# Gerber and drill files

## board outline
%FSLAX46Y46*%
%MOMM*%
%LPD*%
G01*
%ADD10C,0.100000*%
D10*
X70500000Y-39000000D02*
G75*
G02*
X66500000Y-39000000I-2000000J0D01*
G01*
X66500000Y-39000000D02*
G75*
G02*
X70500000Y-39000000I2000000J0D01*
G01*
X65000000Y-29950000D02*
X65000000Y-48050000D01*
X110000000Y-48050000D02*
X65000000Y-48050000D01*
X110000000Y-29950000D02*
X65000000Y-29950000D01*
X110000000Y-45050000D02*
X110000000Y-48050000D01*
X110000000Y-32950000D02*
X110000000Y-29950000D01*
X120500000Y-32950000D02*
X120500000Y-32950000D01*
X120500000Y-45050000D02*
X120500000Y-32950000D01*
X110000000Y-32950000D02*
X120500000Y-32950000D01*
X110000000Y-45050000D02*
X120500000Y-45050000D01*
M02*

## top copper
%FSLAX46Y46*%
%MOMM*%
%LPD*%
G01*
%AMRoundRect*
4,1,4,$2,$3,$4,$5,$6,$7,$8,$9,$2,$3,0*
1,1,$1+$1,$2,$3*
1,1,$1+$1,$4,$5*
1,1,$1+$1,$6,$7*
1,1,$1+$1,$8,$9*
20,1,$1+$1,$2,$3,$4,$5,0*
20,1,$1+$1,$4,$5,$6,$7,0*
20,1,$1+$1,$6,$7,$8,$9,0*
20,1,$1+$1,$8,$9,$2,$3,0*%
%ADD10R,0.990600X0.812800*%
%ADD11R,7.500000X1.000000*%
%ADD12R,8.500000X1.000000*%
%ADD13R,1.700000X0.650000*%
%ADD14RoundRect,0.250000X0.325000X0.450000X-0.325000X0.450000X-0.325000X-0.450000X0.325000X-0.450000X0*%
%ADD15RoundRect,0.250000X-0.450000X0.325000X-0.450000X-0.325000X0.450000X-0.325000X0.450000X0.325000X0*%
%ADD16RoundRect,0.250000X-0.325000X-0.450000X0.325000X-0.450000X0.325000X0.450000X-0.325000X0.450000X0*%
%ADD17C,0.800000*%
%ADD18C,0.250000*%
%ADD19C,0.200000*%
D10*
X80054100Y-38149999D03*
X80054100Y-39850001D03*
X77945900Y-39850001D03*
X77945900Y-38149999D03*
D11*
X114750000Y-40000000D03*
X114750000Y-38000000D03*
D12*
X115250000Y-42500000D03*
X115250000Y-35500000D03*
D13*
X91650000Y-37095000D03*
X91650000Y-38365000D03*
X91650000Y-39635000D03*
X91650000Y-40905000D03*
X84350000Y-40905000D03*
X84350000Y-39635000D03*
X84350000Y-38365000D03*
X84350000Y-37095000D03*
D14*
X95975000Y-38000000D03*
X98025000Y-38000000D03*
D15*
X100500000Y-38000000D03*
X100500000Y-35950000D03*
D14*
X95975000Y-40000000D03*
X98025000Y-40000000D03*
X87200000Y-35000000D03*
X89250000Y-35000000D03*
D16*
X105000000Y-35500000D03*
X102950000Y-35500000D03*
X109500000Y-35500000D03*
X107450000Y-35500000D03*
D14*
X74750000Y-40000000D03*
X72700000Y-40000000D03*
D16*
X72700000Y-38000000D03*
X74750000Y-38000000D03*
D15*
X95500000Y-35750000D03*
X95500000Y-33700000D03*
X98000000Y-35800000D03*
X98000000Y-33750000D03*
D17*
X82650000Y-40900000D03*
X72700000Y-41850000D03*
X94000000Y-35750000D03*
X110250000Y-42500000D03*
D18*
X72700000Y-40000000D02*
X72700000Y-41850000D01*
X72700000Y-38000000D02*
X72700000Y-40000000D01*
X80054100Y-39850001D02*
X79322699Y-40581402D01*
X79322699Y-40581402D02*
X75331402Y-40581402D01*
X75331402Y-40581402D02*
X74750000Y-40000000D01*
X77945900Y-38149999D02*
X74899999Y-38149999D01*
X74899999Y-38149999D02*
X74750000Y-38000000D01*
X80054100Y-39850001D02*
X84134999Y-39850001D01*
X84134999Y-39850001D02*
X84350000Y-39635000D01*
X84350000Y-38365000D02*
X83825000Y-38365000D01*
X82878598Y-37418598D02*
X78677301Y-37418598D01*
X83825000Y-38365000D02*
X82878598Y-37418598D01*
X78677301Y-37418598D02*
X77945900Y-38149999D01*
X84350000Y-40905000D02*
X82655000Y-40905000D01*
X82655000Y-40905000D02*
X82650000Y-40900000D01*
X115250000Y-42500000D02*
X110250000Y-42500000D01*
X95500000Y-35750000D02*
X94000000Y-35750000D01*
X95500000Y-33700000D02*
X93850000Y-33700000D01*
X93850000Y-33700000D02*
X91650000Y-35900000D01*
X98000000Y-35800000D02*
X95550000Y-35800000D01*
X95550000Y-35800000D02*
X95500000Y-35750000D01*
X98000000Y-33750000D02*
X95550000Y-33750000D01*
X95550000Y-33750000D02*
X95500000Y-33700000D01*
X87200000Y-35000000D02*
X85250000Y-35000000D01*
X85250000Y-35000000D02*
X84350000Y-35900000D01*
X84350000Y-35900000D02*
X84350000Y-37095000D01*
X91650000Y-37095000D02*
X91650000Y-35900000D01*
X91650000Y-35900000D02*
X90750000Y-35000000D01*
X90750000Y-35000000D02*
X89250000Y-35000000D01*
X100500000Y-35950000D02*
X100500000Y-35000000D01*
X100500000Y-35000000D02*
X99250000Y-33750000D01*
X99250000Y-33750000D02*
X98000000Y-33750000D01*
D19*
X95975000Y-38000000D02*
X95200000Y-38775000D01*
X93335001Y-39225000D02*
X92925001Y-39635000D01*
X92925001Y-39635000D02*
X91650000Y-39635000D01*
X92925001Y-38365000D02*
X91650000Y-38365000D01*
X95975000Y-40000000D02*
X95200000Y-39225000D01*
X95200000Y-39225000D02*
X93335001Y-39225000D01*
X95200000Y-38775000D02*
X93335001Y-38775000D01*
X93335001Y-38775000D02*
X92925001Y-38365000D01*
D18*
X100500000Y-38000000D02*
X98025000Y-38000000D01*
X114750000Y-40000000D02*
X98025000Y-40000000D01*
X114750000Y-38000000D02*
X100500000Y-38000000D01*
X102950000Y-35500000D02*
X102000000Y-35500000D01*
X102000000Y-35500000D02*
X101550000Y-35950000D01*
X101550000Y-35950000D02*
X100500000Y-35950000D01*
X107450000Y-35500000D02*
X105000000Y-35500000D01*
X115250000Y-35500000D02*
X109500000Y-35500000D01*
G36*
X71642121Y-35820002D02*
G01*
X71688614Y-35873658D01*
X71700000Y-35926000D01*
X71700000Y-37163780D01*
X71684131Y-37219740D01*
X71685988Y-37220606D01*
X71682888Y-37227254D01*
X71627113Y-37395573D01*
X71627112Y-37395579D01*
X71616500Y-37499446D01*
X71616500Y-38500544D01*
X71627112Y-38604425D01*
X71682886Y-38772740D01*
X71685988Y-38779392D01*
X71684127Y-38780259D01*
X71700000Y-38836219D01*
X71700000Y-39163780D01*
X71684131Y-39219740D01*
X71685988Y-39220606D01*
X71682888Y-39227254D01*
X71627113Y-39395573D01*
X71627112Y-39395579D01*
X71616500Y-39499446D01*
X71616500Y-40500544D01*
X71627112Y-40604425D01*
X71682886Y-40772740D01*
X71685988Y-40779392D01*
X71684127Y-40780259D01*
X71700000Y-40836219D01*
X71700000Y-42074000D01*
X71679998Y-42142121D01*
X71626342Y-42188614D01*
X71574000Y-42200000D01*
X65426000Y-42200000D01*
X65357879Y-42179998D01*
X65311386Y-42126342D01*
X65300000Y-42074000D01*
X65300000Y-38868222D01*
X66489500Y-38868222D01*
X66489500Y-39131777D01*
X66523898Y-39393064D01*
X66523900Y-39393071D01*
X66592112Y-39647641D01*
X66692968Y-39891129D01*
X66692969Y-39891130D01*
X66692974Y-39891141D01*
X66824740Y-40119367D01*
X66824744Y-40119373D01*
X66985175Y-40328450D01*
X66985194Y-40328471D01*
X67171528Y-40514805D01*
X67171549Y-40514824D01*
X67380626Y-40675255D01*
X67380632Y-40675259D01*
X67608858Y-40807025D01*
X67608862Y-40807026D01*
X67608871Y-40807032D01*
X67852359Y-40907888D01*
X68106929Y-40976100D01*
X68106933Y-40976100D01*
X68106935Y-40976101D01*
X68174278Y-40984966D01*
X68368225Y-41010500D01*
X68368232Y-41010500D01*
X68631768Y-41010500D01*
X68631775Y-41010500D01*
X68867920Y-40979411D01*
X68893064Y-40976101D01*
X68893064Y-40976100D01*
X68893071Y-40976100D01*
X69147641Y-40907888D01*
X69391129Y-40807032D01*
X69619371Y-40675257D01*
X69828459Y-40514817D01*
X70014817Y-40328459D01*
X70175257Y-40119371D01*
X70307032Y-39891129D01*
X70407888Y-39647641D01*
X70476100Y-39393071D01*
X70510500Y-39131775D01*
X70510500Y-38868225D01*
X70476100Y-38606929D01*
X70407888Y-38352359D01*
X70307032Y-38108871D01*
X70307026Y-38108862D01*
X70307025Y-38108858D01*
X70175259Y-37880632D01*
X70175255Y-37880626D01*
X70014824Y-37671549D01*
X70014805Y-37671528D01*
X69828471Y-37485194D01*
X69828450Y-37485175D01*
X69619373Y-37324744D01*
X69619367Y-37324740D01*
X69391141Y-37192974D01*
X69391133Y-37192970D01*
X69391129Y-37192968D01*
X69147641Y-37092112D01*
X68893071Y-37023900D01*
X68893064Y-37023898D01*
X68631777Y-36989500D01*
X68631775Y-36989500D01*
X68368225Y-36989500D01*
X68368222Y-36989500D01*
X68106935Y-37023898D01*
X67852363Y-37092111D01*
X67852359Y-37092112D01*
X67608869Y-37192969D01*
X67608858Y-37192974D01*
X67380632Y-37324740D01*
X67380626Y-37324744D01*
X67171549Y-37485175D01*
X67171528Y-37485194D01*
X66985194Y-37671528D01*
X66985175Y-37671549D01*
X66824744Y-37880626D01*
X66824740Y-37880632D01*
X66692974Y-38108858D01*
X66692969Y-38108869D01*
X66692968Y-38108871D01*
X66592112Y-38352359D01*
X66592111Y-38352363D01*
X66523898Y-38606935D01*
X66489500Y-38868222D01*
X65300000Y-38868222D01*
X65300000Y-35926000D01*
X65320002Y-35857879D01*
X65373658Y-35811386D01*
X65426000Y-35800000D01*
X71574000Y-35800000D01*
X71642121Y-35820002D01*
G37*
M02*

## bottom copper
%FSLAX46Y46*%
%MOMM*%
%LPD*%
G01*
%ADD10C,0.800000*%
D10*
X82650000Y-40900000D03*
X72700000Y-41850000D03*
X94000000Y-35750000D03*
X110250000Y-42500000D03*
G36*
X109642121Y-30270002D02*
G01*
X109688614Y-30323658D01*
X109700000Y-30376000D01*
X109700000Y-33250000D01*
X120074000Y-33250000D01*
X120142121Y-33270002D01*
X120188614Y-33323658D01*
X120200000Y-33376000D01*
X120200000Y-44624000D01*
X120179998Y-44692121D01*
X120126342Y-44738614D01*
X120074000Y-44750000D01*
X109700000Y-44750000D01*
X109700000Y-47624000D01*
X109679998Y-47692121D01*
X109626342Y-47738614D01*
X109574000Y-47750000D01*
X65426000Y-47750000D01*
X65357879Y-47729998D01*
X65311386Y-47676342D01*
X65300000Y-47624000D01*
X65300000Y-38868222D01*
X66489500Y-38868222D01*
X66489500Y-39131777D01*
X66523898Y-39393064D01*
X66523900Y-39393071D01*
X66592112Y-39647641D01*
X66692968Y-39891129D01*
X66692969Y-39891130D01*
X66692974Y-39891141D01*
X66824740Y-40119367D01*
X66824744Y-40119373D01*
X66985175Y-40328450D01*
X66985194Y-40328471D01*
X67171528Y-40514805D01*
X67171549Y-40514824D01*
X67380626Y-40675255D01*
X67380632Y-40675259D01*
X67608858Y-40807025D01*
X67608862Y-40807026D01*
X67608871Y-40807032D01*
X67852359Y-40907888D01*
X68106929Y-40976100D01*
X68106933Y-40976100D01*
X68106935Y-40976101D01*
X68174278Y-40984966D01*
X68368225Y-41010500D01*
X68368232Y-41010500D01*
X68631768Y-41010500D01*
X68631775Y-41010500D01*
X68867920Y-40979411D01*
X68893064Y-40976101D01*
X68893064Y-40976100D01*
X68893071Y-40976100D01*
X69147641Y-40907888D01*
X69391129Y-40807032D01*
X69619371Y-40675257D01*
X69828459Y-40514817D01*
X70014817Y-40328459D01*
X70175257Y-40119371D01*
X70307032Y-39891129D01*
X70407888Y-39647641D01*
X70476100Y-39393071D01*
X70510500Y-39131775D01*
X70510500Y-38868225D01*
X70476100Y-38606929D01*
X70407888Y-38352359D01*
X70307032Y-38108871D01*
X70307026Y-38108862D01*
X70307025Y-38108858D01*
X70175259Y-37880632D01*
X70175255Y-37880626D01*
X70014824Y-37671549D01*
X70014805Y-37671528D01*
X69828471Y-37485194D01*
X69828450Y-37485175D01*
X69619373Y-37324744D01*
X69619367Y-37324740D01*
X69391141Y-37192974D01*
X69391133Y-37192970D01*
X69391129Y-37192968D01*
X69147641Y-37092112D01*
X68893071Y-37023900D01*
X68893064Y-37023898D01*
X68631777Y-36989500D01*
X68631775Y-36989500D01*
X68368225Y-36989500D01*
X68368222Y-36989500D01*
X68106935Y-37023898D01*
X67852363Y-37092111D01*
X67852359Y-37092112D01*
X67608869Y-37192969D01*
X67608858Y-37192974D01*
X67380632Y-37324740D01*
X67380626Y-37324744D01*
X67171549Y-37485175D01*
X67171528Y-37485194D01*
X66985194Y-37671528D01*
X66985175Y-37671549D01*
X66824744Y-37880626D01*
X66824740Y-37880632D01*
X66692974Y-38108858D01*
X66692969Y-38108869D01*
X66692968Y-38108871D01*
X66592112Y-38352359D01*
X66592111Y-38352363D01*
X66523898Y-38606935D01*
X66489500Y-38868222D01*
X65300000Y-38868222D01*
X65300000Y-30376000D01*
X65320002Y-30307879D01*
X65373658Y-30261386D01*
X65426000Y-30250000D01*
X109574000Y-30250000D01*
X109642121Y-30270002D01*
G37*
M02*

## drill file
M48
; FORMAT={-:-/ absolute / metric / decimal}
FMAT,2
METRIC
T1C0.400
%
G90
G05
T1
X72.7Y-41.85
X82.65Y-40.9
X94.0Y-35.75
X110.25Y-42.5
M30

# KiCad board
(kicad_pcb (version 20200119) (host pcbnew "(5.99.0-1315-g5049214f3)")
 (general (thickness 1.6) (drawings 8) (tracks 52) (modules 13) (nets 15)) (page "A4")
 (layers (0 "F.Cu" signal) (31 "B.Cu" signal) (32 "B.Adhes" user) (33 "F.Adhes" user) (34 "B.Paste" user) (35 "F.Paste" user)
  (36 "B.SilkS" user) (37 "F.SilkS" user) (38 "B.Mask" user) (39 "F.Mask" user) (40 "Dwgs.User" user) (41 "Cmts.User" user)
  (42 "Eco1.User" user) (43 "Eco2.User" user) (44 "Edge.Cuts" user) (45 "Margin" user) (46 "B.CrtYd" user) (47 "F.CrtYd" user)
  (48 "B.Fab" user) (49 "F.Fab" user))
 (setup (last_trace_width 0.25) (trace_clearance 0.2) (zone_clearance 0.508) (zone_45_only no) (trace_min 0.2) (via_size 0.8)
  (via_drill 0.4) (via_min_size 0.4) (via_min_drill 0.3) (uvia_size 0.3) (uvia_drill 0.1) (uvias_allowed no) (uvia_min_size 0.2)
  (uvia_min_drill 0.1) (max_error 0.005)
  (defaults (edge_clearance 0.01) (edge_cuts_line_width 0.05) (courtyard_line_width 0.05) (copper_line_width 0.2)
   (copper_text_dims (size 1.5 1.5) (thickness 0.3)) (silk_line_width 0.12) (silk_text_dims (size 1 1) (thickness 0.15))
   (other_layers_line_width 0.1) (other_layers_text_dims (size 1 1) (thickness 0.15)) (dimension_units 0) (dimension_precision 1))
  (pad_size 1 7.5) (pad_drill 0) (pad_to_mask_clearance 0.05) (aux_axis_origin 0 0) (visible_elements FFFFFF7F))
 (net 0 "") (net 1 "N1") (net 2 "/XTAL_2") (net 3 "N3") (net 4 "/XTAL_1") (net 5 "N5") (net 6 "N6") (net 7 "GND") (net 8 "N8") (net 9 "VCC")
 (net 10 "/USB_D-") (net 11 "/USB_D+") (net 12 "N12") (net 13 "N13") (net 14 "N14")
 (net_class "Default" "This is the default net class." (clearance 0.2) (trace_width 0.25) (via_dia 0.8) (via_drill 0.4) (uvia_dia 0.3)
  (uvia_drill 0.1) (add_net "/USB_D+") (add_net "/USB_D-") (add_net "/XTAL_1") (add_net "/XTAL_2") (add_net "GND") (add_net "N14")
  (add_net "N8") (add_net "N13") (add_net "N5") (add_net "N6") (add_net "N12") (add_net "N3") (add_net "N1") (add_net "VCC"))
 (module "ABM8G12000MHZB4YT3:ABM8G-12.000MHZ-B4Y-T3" (layer "F.Cu") (at 79 39)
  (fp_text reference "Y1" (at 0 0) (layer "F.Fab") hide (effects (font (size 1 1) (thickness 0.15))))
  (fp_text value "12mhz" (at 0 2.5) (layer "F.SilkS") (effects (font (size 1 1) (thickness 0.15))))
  (pad "4" smd rect (at 1.0541 -0.850001 90) (size 0.8128 0.9906) (layers "F.Cu" "F.Paste" "F.Mask") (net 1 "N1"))
  (pad "3" smd rect (at 1.0541 0.850001 90) (size 0.8128 0.9906) (layers "F.Cu" "F.Paste" "F.Mask") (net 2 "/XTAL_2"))
  (pad "2" smd rect (at -1.0541 0.850001 90) (size 0.8128 0.9906) (layers "F.Cu" "F.Paste" "F.Mask") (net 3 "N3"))
  (pad "1" smd rect (at -1.0541 -0.850001 90) (size 0.8128 0.9906) (layers "F.Cu" "F.Paste" "F.Mask") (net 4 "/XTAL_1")))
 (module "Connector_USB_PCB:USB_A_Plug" (layer "F.Cu") (at 115.25 39 90)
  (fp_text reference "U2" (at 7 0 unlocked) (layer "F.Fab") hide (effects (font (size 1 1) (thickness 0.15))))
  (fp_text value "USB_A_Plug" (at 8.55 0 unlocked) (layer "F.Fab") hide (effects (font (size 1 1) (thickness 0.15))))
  (fp_line (start 6.05 5.25) (end 6.05 5.25) (layer "Edge.Cuts") (width 0.1))
  (fp_line (start -6.05 5.25) (end 6.05 5.25) (layer "Edge.Cuts") (width 0.1))
  (fp_line (start 6.05 -5.25) (end 6.05 5.25) (layer "Edge.Cuts") (width 0.1))
  (fp_line (start -6.05 -5.25) (end -6.05 5.25) (layer "Edge.Cuts") (width 0.1))
  (pad "3" smd rect (at -1 -0.5 90) (size 1 7.5) (layers "F.Cu" "F.Paste" "F.Mask") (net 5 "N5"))
  (pad "2" smd rect (at 1 -0.5 90) (size 1 7.5) (layers "F.Cu" "F.Paste" "F.Mask") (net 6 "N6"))
  (pad "4" smd rect (at -3.5 0 90) (size 1 8.5) (layers "F.Cu" "F.Paste" "F.Mask") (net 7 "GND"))
  (pad "1" smd rect (at 3.5 0 90) (size 1 8.5) (layers "F.Cu" "F.Paste" "F.Mask") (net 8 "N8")))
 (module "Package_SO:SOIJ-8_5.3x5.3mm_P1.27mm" (layer "F.Cu") (at 88 39)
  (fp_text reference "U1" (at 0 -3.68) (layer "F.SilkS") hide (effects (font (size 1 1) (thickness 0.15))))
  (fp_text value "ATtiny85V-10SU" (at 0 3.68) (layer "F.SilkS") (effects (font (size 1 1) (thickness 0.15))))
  (pad "8" smd rect (at 3.65 -1.905) (size 1.7 0.65) (layers "F.Cu" "F.Paste" "F.Mask") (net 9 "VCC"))
  (pad "7" smd rect (at 3.65 -0.635) (size 1.7 0.65) (layers "F.Cu" "F.Paste" "F.Mask") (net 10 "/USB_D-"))
  (pad "6" smd rect (at 3.65 0.635) (size 1.7 0.65) (layers "F.Cu" "F.Paste" "F.Mask") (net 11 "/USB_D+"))
  (pad "5" smd rect (at 3.65 1.905) (size 1.7 0.65) (layers "F.Cu" "F.Paste" "F.Mask") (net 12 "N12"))
  (pad "4" smd rect (at -3.65 1.905) (size 1.7 0.65) (layers "F.Cu" "F.Paste" "F.Mask") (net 7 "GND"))
  (pad "3" smd rect (at -3.65 0.635) (size 1.7 0.65) (layers "F.Cu" "F.Paste" "F.Mask") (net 2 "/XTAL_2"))
  (pad "2" smd rect (at -3.65 -0.635) (size 1.7 0.65) (layers "F.Cu" "F.Paste" "F.Mask") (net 4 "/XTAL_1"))
  (pad "1" smd rect (at -3.65 -1.905) (size 1.7 0.65) (layers "F.Cu" "F.Paste" "F.Mask") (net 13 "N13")))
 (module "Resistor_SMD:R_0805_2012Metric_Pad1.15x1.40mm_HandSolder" (layer "F.Cu") (at 97 38 180)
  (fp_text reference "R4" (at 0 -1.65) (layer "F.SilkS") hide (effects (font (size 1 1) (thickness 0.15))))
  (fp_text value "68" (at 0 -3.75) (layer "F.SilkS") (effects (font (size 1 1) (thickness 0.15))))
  (pad "2" smd roundrect (at 1.025 0 180) (size 1.15 1.4) (layers "F.Cu" "F.Paste" "F.Mask") (roundrect_rratio 0.217391) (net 10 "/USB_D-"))
  (pad "1" smd roundrect (at -1.025 0 180) (size 1.15 1.4) (layers "F.Cu" "F.Paste" "F.Mask") (roundrect_rratio 0.217391) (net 6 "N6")))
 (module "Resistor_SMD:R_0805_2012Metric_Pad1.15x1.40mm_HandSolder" (layer "F.Cu") (at 100.5 36.975 -90)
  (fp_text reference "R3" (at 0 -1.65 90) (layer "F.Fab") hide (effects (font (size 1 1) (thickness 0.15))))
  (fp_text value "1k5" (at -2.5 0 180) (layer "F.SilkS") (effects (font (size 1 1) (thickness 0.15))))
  (pad "2" smd roundrect (at 1.025 0 270) (size 1.15 1.4) (layers "F.Cu" "F.Paste" "F.Mask") (roundrect_rratio 0.217391) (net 6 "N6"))
  (pad "1" smd roundrect (at -1.025 0 270) (size 1.15 1.4) (layers "F.Cu" "F.Paste" "F.Mask") (roundrect_rratio 0.217391) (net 9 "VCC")))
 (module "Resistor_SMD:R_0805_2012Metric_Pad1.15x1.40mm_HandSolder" (layer "F.Cu") (at 97 40 180)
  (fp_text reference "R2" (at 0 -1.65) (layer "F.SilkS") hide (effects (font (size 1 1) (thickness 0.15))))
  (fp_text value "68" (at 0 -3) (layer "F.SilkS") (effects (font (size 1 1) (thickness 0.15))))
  (pad "2" smd roundrect (at 1.025 0 180) (size 1.15 1.4) (layers "F.Cu" "F.Paste" "F.Mask") (roundrect_rratio 0.217391) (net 11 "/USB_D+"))
  (pad "1" smd roundrect (at -1.025 0 180) (size 1.15 1.4) (layers "F.Cu" "F.Paste" "F.Mask") (roundrect_rratio 0.217391) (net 5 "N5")))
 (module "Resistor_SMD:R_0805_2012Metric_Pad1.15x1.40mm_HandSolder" (layer "F.Cu") (at 88.225 35 180)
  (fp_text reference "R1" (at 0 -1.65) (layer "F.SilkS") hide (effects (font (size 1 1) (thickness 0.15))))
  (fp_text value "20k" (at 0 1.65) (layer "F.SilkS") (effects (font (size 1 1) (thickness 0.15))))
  (pad "2" smd roundrect (at 1.025 0 180) (size 1.15 1.4) (layers "F.Cu" "F.Paste" "F.Mask") (roundrect_rratio 0.217391) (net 13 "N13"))
  (pad "1" smd roundrect (at -1.025 0 180) (size 1.15 1.4) (layers "F.Cu" "F.Paste" "F.Mask") (roundrect_rratio 0.217391) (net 9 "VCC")))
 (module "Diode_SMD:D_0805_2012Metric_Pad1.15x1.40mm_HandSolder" (layer "F.Cu") (at 103.975 35.5)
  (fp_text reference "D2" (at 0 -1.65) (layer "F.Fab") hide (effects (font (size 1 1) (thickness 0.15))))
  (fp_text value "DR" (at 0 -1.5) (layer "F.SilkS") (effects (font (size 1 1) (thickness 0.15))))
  (pad "2" smd roundrect (at 1.025 0) (size 1.15 1.4) (layers "F.Cu" "F.Paste" "F.Mask") (roundrect_rratio 0.217391) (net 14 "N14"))
  (pad "1" smd roundrect (at -1.025 0) (size 1.15 1.4) (layers "F.Cu" "F.Paste" "F.Mask") (roundrect_rratio 0.217391) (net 9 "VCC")))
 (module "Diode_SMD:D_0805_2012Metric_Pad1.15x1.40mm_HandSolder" (layer "F.Cu") (at 108.475 35.5)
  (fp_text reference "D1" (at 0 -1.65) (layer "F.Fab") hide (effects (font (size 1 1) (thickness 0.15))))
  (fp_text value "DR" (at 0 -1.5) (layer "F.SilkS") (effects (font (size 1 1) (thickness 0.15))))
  (pad "2" smd roundrect (at 1.025 0) (size 1.15 1.4) (layers "F.Cu" "F.Paste" "F.Mask") (roundrect_rratio 0.217391) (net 8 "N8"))
  (pad "1" smd roundrect (at -1.025 0) (size 1.15 1.4) (layers "F.Cu" "F.Paste" "F.Mask") (roundrect_rratio 0.217391) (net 14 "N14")))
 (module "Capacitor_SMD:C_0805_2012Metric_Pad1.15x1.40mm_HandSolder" (layer "F.Cu") (at 73.725 40 180)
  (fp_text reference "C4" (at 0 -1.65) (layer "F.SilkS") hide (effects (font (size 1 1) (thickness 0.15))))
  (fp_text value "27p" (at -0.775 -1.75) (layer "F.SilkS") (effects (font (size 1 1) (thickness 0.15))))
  (pad "1" smd roundrect (at -1.025 0 180) (size 1.15 1.4) (layers "F.Cu" "F.Paste" "F.Mask") (roundrect_rratio 0.217391) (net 2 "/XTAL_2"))
  (pad "2" smd roundrect (at 1.025 0 180) (size 1.15 1.4) (layers "F.Cu" "F.Paste" "F.Mask") (roundrect_rratio 0.217391) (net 7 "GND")))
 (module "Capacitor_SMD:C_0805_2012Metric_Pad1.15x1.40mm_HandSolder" (layer "F.Cu") (at 73.725 38)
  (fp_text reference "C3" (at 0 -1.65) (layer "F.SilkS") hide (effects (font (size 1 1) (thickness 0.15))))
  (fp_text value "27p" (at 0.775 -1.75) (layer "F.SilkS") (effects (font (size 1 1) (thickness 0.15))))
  (pad "1" smd roundrect (at -1.025 0) (size 1.15 1.4) (layers "F.Cu" "F.Paste" "F.Mask") (roundrect_rratio 0.217391) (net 7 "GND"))
  (pad "2" smd roundrect (at 1.025 0) (size 1.15 1.4) (layers "F.Cu" "F.Paste" "F.Mask") (roundrect_rratio 0.217391) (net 4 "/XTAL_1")))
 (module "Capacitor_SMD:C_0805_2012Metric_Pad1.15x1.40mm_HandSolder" (layer "F.Cu") (at 95.5 34.725 -90)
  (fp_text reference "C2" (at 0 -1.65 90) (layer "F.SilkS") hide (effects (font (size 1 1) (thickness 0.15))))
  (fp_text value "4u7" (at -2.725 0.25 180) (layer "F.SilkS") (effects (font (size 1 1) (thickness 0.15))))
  (pad "2" smd roundrect (at 1.025 0 270) (size 1.15 1.4) (layers "F.Cu" "F.Paste" "F.Mask") (roundrect_rratio 0.217391) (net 7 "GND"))
  (pad "1" smd roundrect (at -1.025 0 270) (size 1.15 1.4) (layers "F.Cu" "F.Paste" "F.Mask") (roundrect_rratio 0.217391) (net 9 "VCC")))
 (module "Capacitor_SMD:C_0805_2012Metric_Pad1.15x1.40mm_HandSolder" (layer "F.Cu") (at 98 34.775 -90)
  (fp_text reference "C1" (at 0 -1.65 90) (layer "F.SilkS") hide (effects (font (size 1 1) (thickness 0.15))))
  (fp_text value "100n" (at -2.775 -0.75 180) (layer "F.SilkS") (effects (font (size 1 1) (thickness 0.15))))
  (pad "2" smd roundrect (at 1.025 0 270) (size 1.15 1.4) (layers "F.Cu" "F.Paste" "F.Mask") (roundrect_rratio 0.217391) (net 7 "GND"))
  (pad "1" smd roundrect (at -1.025 0 270) (size 1.15 1.4) (layers "F.Cu" "F.Paste" "F.Mask") (roundrect_rratio 0.217391) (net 9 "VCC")))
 (gr_circle (center 68.5 39) (end 70.5 39) (layer "Edge.Cuts") (width 0.1))
 (gr_line (start 65 29.95) (end 65 48.05) (layer "Edge.Cuts") (width 0.1))
 (gr_line (start 110 48.05) (end 65 48.05) (layer "Edge.Cuts") (width 0.1))
 (gr_line (start 110 29.95) (end 65 29.95) (layer "Edge.Cuts") (width 0.1))
 (gr_line (start 110 45.05) (end 110 48.05) (layer "Edge.Cuts") (width 0.1))
 (gr_line (start 110 32.95) (end 110 29.95) (layer "Edge.Cuts") (width 0.1))
 (segment (start 72.7 40) (end 72.7 41.85) (width 0.25) (layer "F.Cu") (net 7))
 (segment (start 72.7 38) (end 72.7 40) (width 0.25) (layer "F.Cu") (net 7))
 (segment (start 80.0541 39.850001) (end 79.322699 40.581402) (width 0.25) (layer "F.Cu") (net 2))
 (segment (start 79.322699 40.581402) (end 75.331402 40.581402) (width 0.25) (layer "F.Cu") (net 2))
 (segment (start 75.331402 40.581402) (end 74.75 40) (width 0.25) (layer "F.Cu") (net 2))
 (segment (start 77.9459 38.149999) (end 74.899999 38.149999) (width 0.25) (layer "F.Cu") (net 4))
 (segment (start 74.899999 38.149999) (end 74.75 38) (width 0.25) (layer "F.Cu") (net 4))
 (segment (start 80.0541 39.850001) (end 84.134999 39.850001) (width 0.25) (layer "F.Cu") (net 2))
 (segment (start 84.134999 39.850001) (end 84.35 39.635) (width 0.25) (layer "F.Cu") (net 2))
 (segment (start 84.35 38.365) (end 83.825 38.365) (width 0.25) (layer "F.Cu") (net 4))
 (segment (start 82.878598 37.418598) (end 78.677301 37.418598) (width 0.25) (layer "F.Cu") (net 4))
 (segment (start 83.825 38.365) (end 82.878598 37.418598) (width 0.25) (layer "F.Cu") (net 4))
 (segment (start 78.677301 37.418598) (end 77.9459 38.149999) (width 0.25) (layer "F.Cu") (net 4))
 (segment (start 84.35 40.905) (end 82.655 40.905) (width 0.25) (layer "F.Cu") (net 7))
 (segment (start 82.655 40.905) (end 82.65 40.9) (width 0.25) (layer "F.Cu") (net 7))
 (via (at 82.65 40.9) (size 0.8) (drill 0.4) (layers "F.Cu" "B.Cu") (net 7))
 (segment (start 115.25 42.5) (end 110.25 42.5) (width 0.25) (layer "F.Cu") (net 7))
 (via (at 72.7 41.85) (size 0.8) (drill 0.4) (layers "F.Cu" "B.Cu") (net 7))
 (segment (start 95.5 35.75) (end 94 35.75) (width 0.25) (layer "F.Cu") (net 7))
 (via (at 94 35.75) (size 0.8) (drill 0.4) (layers "F.Cu" "B.Cu") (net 7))
 (via (at 110.25 42.5) (size 0.8) (drill 0.4) (layers "F.Cu" "B.Cu") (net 7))
 (segment (start 95.5 33.7) (end 93.85 33.7) (width 0.25) (layer "F.Cu") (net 9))
 (segment (start 93.85 33.7) (end 91.65 35.9) (width 0.25) (layer "F.Cu") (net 9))
 (segment (start 98 35.8) (end 95.55 35.8) (width 0.25) (layer "F.Cu") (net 7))
 (segment (start 95.55 35.8) (end 95.5 35.75) (width 0.25) (layer "F.Cu") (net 7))
 (segment (start 98 33.75) (end 95.55 33.75) (width 0.25) (layer "F.Cu") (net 9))
 (segment (start 95.55 33.75) (end 95.5 33.7) (width 0.25) (layer "F.Cu") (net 9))
 (segment (start 87.2 35) (end 85.25 35) (width 0.25) (layer "F.Cu") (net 13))
 (segment (start 85.25 35) (end 84.35 35.9) (width 0.25) (layer "F.Cu") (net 13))
 (segment (start 84.35 35.9) (end 84.35 37.095) (width 0.25) (layer "F.Cu") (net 13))
 (segment (start 91.65 37.095) (end 91.65 35.9) (width 0.25) (layer "F.Cu") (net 9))
 (segment (start 91.65 35.9) (end 90.75 35) (width 0.25) (layer "F.Cu") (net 9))
 (segment (start 90.75 35) (end 89.25 35) (width 0.25) (layer "F.Cu") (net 9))
 (segment (start 100.5 35.95) (end 100.5 35) (width 0.25) (layer "F.Cu") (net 9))
 (segment (start 100.5 35) (end 99.25 33.75) (width 0.25) (layer "F.Cu") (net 9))
 (segment (start 99.25 33.75) (end 98 33.75) (width 0.25) (layer "F.Cu") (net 9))
 (segment (start 95.975 38) (end 95.2 38.775) (width 0.2) (layer "F.Cu") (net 10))
 (segment (start 93.335001 39.225) (end 92.925001 39.635) (width 0.2) (layer "F.Cu") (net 11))
 (segment (start 92.925001 39.635) (end 91.65 39.635) (width 0.2) (layer "F.Cu") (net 11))
 (segment (start 92.925001 38.365) (end 91.65 38.365) (width 0.2) (layer "F.Cu") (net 10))
 (segment (start 95.975 40) (end 95.2 39.225) (width 0.2) (layer "F.Cu") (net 11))
 (segment (start 95.2 39.225) (end 93.335001 39.225) (width 0.2) (layer "F.Cu") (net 11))
 (segment (start 95.2 38.775) (end 93.335001 38.775) (width 0.2) (layer "F.Cu") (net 10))
 (segment (start 93.335001 38.775) (end 92.925001 38.365) (width 0.2) (layer "F.Cu") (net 10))
 (segment (start 100.5 38) (end 98.025 38) (width 0.25) (layer "F.Cu") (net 6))
 (segment (start 114.75 40) (end 98.025 40) (width 0.25) (layer "F.Cu") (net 5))
 (segment (start 114.75 38) (end 100.5 38) (width 0.25) (layer "F.Cu") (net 6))
 (segment (start 102.95 35.5) (end 102 35.5) (width 0.25) (layer "F.Cu") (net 9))
 (segment (start 102 35.5) (end 101.55 35.95) (width 0.25) (layer "F.Cu") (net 9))
 (segment (start 101.55 35.95) (end 100.5 35.95) (width 0.25) (layer "F.Cu") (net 9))
 (segment (start 107.45 35.5) (end 105 35.5) (width 0.25) (layer "F.Cu") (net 14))
 (segment (start 115.25 35.5) (end 109.5 35.5) (width 0.25) (layer "F.Cu") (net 8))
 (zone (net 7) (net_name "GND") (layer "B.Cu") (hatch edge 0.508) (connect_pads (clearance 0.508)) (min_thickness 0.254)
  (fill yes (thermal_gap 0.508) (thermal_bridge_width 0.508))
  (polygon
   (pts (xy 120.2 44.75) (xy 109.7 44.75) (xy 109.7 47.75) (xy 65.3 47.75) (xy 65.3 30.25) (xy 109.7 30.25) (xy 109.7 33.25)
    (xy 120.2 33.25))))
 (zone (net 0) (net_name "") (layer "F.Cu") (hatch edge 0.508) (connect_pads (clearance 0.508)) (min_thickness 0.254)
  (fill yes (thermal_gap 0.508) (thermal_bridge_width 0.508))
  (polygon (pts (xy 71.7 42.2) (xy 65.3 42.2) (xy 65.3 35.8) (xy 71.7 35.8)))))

